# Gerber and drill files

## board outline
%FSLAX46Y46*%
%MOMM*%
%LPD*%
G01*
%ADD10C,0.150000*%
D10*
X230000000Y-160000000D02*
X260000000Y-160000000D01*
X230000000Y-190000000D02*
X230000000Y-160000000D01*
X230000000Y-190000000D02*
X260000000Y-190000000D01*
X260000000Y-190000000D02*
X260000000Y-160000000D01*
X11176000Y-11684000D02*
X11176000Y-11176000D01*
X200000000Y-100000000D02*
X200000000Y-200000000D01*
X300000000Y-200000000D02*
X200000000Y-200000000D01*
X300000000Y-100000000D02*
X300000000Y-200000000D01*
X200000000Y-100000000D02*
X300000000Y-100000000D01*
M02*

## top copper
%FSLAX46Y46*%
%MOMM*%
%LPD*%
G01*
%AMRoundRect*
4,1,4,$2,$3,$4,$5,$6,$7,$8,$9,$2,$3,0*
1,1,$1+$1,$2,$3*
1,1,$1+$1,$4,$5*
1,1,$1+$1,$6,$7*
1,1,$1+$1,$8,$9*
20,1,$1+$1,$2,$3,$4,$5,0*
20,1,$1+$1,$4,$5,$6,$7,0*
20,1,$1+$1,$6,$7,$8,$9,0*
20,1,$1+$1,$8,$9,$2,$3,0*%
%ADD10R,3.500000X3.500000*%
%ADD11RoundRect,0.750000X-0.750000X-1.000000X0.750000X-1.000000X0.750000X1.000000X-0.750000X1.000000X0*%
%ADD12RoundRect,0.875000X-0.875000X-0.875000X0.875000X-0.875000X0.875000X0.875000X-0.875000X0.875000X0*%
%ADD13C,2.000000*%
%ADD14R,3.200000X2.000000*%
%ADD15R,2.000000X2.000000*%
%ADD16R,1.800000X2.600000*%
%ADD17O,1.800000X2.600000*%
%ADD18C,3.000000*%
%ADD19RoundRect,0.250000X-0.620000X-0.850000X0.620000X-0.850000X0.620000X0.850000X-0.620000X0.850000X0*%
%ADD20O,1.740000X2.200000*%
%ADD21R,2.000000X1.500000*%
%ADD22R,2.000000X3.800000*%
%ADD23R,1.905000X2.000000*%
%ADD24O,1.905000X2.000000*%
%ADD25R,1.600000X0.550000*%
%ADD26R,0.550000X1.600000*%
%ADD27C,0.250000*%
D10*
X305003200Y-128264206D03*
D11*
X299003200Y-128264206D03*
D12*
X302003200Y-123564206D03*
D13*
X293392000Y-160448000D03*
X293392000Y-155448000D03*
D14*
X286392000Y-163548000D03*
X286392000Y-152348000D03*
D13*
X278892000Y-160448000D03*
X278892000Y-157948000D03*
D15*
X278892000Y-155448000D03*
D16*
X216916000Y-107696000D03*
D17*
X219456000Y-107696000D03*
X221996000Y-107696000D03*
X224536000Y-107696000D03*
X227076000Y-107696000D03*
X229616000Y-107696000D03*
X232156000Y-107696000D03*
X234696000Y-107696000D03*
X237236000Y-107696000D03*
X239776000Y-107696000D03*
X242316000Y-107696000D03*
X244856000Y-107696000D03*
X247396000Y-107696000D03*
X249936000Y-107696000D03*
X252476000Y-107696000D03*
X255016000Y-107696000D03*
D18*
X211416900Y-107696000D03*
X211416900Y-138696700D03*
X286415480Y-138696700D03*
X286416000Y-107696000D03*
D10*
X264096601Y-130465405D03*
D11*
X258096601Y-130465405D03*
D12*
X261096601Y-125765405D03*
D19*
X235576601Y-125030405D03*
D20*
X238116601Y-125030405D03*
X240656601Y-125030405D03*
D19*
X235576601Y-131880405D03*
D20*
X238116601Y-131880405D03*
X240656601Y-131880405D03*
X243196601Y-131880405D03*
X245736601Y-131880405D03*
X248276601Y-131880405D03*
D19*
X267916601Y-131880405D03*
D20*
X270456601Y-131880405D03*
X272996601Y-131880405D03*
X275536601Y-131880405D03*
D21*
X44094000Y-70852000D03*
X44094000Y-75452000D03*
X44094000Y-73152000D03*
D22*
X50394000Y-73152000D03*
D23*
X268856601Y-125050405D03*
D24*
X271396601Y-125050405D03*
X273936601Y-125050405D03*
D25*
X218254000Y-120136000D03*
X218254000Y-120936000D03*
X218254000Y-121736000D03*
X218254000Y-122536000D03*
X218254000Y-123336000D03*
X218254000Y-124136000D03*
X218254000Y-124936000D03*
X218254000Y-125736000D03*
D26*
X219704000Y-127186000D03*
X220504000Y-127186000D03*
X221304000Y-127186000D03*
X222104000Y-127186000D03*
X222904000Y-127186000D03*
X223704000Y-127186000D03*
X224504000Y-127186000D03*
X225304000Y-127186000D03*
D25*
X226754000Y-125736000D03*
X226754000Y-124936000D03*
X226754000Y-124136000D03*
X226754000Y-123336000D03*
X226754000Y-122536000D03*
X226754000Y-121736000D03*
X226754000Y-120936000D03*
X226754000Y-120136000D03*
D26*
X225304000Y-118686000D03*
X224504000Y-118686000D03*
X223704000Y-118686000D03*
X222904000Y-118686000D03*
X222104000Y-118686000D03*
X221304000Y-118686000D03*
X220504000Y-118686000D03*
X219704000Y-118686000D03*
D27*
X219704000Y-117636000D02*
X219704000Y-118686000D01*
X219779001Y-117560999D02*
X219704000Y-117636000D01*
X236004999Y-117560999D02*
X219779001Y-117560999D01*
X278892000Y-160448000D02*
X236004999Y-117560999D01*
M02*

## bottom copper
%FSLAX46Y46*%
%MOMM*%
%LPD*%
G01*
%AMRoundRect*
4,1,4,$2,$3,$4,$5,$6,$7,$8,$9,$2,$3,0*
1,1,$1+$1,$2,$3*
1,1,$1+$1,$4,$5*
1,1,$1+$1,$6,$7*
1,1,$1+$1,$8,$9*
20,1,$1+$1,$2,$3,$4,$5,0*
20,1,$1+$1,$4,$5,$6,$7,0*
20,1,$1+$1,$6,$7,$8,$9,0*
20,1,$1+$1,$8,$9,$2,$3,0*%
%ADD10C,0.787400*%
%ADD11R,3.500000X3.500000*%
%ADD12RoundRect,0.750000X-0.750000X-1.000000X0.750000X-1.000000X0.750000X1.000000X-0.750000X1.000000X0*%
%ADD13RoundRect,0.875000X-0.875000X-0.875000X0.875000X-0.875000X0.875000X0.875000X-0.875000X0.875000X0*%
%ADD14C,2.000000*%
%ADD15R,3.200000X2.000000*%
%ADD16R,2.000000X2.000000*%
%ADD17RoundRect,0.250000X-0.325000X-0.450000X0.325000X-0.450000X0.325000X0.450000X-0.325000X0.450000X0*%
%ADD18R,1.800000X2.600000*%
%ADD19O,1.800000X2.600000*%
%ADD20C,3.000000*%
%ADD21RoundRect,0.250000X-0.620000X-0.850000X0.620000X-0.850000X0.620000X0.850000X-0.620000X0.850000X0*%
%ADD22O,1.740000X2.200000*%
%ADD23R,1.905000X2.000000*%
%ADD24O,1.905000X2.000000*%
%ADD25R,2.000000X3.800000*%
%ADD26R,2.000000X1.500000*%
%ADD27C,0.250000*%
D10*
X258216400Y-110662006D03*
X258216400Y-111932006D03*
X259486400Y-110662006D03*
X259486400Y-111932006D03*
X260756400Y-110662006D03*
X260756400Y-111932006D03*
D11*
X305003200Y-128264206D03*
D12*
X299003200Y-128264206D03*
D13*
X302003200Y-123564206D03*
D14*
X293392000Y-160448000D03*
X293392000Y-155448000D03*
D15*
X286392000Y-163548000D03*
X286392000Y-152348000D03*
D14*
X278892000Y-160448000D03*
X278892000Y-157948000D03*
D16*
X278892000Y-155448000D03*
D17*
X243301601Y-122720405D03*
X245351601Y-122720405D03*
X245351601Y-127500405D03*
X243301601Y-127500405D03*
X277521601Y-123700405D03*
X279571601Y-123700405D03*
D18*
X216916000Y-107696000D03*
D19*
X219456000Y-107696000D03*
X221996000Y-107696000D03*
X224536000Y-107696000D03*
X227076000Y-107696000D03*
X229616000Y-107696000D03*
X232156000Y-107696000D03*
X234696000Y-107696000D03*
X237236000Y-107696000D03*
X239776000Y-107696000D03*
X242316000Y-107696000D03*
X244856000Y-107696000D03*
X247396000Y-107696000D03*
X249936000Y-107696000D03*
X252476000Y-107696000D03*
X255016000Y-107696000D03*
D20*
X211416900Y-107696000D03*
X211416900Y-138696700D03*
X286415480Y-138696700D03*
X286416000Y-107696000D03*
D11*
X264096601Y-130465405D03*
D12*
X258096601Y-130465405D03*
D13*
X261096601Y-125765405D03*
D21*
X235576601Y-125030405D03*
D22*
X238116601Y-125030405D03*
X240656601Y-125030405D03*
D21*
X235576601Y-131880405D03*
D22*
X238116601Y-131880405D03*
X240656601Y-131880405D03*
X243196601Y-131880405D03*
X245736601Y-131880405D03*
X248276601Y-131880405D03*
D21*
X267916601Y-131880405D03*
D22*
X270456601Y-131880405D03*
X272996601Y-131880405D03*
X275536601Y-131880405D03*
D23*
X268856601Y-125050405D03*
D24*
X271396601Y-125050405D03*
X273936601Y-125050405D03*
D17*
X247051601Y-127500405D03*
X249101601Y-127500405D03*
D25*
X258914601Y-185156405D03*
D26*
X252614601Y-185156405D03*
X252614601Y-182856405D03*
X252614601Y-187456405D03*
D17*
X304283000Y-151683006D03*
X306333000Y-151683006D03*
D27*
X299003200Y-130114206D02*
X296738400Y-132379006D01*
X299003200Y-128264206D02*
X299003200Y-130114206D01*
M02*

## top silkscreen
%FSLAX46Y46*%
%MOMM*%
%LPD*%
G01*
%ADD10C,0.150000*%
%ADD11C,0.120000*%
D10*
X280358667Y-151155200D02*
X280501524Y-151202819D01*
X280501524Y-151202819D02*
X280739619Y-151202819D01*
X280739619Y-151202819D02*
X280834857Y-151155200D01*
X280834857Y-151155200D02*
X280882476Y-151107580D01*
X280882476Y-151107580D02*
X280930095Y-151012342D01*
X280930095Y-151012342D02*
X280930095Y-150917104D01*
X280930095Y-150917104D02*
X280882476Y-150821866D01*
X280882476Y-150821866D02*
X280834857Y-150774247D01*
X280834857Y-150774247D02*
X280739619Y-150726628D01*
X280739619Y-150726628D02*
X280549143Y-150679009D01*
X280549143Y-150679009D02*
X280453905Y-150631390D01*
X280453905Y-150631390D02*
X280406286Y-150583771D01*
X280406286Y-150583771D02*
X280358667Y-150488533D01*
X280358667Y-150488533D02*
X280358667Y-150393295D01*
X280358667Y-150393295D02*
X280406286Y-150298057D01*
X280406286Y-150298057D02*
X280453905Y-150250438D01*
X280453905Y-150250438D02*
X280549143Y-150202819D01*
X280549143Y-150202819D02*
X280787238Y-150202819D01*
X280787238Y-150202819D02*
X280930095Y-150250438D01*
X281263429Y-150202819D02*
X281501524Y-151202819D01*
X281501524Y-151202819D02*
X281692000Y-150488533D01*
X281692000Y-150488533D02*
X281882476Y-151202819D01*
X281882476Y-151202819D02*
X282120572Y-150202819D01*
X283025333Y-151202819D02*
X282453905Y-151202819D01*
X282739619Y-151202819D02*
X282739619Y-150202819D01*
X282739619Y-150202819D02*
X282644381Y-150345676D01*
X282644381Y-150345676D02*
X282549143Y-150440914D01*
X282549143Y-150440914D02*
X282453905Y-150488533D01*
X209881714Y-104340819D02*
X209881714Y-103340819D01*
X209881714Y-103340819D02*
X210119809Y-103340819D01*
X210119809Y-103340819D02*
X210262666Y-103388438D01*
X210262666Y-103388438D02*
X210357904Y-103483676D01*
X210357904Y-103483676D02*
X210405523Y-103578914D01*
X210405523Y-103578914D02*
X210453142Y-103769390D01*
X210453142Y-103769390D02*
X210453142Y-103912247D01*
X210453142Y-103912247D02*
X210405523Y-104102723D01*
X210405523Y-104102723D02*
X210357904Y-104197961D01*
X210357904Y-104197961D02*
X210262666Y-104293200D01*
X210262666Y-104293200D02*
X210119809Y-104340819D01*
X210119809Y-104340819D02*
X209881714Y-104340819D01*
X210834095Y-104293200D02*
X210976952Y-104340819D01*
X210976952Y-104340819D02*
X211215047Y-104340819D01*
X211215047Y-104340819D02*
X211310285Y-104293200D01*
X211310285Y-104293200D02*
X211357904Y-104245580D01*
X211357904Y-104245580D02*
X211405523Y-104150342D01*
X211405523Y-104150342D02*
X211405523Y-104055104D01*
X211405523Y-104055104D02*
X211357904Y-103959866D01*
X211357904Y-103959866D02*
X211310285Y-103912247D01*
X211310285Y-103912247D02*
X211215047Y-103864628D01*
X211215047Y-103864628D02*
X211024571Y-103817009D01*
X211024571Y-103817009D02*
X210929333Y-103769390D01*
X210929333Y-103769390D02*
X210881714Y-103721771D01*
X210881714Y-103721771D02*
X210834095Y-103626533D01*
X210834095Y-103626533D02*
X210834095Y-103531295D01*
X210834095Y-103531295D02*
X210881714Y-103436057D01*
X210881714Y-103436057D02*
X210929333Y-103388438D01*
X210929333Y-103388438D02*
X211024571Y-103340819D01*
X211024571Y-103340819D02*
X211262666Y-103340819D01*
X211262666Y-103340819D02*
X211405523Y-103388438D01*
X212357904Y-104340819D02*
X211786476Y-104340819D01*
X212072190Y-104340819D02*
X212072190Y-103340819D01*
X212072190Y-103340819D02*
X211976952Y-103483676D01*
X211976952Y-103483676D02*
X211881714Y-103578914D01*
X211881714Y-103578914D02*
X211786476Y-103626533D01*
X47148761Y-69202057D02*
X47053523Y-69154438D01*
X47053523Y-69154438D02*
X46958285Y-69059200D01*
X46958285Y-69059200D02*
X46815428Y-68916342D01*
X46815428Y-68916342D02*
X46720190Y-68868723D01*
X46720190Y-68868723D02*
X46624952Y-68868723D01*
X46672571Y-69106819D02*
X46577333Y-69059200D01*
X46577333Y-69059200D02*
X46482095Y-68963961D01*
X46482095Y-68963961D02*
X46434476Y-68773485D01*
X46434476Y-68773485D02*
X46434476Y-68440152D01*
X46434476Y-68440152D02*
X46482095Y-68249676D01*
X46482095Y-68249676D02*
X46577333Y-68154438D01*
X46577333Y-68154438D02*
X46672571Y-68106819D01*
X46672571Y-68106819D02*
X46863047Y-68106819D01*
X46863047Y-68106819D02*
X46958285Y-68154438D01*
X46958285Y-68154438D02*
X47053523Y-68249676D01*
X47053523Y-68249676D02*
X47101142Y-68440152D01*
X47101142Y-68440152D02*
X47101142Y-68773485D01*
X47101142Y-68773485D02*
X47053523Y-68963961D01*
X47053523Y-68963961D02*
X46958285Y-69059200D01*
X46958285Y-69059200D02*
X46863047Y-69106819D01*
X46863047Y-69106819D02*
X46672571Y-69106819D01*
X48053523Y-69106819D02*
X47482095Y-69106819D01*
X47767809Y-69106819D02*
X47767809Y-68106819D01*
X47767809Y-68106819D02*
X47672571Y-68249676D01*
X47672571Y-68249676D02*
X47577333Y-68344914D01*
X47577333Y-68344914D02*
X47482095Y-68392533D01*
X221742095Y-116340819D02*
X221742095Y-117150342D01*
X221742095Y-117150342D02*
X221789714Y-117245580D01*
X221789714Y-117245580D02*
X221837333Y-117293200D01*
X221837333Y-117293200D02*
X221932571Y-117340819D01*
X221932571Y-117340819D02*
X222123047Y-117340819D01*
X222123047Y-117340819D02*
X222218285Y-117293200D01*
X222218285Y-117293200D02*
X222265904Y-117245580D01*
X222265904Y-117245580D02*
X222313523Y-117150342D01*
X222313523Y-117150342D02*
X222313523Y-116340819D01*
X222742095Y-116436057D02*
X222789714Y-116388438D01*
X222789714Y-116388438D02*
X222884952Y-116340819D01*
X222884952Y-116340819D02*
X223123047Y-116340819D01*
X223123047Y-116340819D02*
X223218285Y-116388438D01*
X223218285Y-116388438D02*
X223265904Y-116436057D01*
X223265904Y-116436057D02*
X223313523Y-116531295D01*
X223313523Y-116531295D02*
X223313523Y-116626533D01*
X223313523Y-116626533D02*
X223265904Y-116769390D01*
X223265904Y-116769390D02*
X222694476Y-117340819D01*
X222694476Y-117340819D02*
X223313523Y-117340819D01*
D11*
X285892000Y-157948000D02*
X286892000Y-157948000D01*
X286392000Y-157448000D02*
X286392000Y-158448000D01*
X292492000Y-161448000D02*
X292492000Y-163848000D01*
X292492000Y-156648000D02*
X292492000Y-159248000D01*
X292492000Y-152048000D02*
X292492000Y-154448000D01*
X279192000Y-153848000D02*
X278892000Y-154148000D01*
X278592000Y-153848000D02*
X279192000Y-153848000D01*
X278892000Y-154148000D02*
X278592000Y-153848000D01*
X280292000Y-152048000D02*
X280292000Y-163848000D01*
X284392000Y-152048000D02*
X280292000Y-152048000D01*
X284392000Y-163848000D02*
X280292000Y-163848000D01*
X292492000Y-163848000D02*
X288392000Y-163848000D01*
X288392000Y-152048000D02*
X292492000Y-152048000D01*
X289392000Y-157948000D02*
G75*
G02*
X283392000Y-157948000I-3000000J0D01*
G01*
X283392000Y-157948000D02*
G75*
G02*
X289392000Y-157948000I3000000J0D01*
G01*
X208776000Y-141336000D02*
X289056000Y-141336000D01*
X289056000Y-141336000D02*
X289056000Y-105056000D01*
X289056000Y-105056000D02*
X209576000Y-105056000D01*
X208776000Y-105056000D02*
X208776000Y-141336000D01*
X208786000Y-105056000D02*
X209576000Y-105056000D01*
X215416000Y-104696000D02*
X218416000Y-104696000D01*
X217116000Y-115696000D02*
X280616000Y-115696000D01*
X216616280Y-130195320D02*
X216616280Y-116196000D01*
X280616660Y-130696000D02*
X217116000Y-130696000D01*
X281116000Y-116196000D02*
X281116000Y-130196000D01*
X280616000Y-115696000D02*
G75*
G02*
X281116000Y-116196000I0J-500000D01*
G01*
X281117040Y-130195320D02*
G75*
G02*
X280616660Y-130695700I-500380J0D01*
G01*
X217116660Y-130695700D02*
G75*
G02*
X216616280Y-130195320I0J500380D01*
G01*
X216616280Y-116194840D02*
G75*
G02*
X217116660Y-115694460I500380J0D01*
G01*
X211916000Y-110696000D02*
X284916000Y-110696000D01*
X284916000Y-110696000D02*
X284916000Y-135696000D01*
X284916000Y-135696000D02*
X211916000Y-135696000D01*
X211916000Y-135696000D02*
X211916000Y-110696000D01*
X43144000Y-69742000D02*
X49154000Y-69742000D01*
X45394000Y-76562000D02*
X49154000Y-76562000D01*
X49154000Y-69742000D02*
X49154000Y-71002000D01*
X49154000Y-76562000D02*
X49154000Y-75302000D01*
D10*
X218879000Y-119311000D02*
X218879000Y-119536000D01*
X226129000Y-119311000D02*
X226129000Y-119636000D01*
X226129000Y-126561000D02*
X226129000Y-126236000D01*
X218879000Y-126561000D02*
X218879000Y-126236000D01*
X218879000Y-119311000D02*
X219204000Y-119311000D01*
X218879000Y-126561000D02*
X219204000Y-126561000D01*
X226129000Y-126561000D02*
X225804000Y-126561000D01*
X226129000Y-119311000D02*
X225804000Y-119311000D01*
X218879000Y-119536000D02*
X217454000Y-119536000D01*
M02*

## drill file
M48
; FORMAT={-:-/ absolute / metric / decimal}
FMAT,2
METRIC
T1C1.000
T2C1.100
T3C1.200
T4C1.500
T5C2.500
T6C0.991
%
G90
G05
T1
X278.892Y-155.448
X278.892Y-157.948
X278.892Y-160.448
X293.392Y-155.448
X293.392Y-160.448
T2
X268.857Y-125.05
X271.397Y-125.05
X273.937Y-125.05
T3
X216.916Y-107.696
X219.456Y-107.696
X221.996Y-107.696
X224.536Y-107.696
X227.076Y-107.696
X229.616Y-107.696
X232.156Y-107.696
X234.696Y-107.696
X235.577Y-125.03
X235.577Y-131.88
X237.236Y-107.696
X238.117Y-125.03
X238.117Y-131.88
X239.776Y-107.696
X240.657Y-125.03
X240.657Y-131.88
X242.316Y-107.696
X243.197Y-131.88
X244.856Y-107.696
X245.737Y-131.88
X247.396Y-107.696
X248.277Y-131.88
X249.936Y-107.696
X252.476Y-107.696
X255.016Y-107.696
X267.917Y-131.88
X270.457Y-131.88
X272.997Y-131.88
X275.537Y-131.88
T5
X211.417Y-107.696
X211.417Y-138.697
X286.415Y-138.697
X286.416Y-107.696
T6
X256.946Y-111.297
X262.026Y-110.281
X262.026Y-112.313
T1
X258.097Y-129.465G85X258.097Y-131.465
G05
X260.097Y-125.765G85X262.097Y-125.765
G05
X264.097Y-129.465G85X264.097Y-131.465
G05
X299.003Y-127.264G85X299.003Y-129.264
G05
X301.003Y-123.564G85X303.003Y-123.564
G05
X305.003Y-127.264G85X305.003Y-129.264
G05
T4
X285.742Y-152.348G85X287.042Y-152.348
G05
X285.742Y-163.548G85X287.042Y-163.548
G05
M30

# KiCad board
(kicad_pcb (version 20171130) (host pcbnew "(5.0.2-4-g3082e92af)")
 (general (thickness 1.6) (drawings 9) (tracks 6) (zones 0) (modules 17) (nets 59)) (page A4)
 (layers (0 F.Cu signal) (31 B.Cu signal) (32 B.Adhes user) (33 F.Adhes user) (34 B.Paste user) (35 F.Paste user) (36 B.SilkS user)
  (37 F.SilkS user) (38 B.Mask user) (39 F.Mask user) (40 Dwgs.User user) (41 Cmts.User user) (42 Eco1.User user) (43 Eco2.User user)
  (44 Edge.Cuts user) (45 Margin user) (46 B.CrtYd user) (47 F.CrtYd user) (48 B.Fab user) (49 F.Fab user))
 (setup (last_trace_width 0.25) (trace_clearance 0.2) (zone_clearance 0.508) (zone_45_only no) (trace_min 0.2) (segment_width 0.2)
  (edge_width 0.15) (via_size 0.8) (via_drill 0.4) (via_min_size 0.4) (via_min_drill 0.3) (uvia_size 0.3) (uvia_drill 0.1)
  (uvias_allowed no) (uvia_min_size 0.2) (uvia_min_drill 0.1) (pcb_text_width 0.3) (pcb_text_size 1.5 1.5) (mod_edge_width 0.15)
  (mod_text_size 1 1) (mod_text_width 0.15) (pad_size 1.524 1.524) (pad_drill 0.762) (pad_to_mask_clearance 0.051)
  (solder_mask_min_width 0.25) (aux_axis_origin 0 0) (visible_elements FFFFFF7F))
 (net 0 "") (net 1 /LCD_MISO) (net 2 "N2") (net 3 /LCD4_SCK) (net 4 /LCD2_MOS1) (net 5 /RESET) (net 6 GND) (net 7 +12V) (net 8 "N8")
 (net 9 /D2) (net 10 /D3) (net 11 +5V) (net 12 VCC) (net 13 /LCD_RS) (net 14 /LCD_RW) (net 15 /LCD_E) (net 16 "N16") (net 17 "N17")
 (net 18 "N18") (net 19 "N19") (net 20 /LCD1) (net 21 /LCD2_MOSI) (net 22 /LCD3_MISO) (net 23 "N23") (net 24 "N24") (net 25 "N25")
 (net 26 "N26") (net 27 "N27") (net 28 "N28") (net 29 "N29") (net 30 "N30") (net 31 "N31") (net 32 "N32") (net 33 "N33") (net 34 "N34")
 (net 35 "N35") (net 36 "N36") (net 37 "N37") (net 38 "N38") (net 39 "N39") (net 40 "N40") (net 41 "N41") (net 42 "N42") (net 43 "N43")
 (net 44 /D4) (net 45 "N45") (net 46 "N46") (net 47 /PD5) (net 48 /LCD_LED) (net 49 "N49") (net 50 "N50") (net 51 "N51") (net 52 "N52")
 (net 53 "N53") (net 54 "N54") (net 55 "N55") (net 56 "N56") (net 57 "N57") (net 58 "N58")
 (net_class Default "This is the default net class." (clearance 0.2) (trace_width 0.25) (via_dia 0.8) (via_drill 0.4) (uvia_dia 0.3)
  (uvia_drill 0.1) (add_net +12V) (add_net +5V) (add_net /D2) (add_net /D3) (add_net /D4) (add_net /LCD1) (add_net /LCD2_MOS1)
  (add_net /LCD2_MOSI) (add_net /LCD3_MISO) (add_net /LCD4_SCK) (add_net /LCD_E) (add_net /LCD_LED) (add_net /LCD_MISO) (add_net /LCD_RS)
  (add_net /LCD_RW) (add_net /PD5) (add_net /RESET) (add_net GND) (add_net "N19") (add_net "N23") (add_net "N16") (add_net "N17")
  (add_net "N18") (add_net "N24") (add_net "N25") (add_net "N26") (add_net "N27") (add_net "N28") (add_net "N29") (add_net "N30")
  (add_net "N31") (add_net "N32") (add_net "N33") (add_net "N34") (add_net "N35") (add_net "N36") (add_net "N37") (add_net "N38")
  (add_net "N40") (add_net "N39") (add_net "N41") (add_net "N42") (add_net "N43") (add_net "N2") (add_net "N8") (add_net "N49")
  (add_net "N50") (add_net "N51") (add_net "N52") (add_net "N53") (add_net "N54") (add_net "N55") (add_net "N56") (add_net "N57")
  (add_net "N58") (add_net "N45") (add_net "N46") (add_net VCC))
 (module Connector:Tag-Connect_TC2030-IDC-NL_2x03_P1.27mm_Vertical (layer B.Cu) (at 259.4864 111.297006)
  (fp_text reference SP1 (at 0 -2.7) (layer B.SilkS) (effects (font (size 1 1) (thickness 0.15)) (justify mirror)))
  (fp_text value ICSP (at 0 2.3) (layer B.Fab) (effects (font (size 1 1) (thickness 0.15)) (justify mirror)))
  (pad "" np_thru_hole circle (at 2.54 1.016) (size 0.9906 0.9906) (drill 0.9906) (layers *.Cu *.Mask))
  (pad "" np_thru_hole circle (at 2.54 -1.016) (size 0.9906 0.9906) (drill 0.9906) (layers *.Cu *.Mask))
  (pad "" np_thru_hole circle (at -2.54 0) (size 0.9906 0.9906) (drill 0.9906) (layers *.Cu *.Mask))
  (pad 1 connect circle (at -1.27 -0.635) (size 0.7874 0.7874) (layers B.Cu B.Mask) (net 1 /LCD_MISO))
  (pad 2 connect circle (at -1.27 0.635) (size 0.7874 0.7874) (layers B.Cu B.Mask) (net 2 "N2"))
  (pad 3 connect circle (at 0 -0.635) (size 0.7874 0.7874) (layers B.Cu B.Mask) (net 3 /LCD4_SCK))
  (pad 4 connect circle (at 0 0.635) (size 0.7874 0.7874) (layers B.Cu B.Mask) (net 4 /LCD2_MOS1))
  (pad 5 connect circle (at 1.27 -0.635) (size 0.7874 0.7874) (layers B.Cu B.Mask) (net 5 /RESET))
  (pad 6 connect circle (at 1.27 0.635) (size 0.7874 0.7874) (layers B.Cu B.Mask) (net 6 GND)))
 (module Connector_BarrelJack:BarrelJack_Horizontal (layer B.Cu) (at 305.0032 128.264206)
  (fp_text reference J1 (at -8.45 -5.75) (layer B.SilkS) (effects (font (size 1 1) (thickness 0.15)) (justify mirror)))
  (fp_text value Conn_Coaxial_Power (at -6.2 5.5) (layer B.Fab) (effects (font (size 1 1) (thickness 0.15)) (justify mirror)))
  (pad 1 thru_hole rect (at 0 0) (size 3.5 3.5) (drill oval 1 3) (layers *.Cu *.Mask) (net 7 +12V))
  (pad 2 thru_hole roundrect (at -6 0) (size 3 3.5) (drill oval 1 3) (layers *.Cu *.Mask) (roundrect_rratio 0.25) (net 6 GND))
  (pad 3 thru_hole roundrect (at -3 -4.7) (size 3.5 3.5) (drill oval 3 1) (layers *.Cu *.Mask) (roundrect_rratio 0.25)))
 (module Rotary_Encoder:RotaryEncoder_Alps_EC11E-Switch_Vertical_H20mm (layer F.Cu) (at 278.892 155.448)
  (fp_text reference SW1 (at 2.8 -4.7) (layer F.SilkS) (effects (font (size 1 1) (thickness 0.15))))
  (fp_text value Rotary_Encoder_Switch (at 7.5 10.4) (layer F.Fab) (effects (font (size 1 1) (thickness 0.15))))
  (fp_line (start 7 2.5) (end 8 2.5) (layer F.SilkS) (width 0.12))
  (fp_line (start 7.5 2) (end 7.5 3) (layer F.SilkS) (width 0.12))
  (fp_line (start 13.6 6) (end 13.6 8.4) (layer F.SilkS) (width 0.12))
  (fp_line (start 13.6 1.2) (end 13.6 3.8) (layer F.SilkS) (width 0.12))
  (fp_line (start 13.6 -3.4) (end 13.6 -1) (layer F.SilkS) (width 0.12))
  (fp_line (start 0.3 -1.6) (end 0 -1.3) (layer F.SilkS) (width 0.12))
  (fp_line (start -0.3 -1.6) (end 0.3 -1.6) (layer F.SilkS) (width 0.12))
  (fp_line (start 0 -1.3) (end -0.3 -1.6) (layer F.SilkS) (width 0.12))
  (fp_line (start 1.4 -3.4) (end 1.4 8.4) (layer F.SilkS) (width 0.12))
  (fp_line (start 5.5 -3.4) (end 1.4 -3.4) (layer F.SilkS) (width 0.12))
  (fp_line (start 5.5 8.4) (end 1.4 8.4) (layer F.SilkS) (width 0.12))
  (fp_line (start 13.6 8.4) (end 9.5 8.4) (layer F.SilkS) (width 0.12))
  (fp_line (start 9.5 -3.4) (end 13.6 -3.4) (layer F.SilkS) (width 0.12))
  (fp_circle (center 7.5 2.5) (end 10.5 2.5) (layer F.SilkS) (width 0.12))
  (pad S1 thru_hole circle (at 14.5 5) (size 2 2) (drill 1) (layers *.Cu *.Mask) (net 6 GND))
  (pad S2 thru_hole circle (at 14.5 0) (size 2 2) (drill 1) (layers *.Cu *.Mask) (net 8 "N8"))
  (pad MP thru_hole rect (at 7.5 8.1) (size 3.2 2) (drill oval 2.8 1.5) (layers *.Cu *.Mask))
  (pad MP thru_hole rect (at 7.5 -3.1) (size 3.2 2) (drill oval 2.8 1.5) (layers *.Cu *.Mask))
  (pad B thru_hole circle (at 0 5) (size 2 2) (drill 1) (layers *.Cu *.Mask) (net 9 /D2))
  (pad C thru_hole circle (at 0 2.5) (size 2 2) (drill 1) (layers *.Cu *.Mask) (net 6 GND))
  (pad A thru_hole rect (at 0 0) (size 2 2) (drill 1) (layers *.Cu *.Mask) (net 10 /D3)))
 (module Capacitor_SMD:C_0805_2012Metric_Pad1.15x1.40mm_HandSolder (layer B.Cu) (at 244.326601 122.720405)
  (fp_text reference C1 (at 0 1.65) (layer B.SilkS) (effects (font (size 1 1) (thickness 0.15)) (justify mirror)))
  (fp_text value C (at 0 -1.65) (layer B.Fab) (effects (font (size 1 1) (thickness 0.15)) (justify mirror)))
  (pad 1 smd roundrect (at -1.025 0) (size 1.15 1.4) (layers B.Cu B.Paste B.Mask) (roundrect_rratio 0.217391) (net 7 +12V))
  (pad 2 smd roundrect (at 1.025 0) (size 1.15 1.4) (layers B.Cu B.Paste B.Mask) (roundrect_rratio 0.217391) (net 6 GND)))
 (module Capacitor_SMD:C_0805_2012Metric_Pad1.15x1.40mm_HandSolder (layer B.Cu) (at 244.326601 127.500405)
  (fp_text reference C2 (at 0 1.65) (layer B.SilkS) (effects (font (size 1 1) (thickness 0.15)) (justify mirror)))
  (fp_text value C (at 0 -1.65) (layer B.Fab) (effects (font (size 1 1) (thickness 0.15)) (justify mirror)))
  (pad 2 smd roundrect (at 1.025 0) (size 1.15 1.4) (layers B.Cu B.Paste B.Mask) (roundrect_rratio 0.217391) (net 6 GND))
  (pad 1 smd roundrect (at -1.025 0) (size 1.15 1.4) (layers B.Cu B.Paste B.Mask) (roundrect_rratio 0.217391) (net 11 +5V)))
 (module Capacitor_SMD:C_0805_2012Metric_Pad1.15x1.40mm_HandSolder (layer B.Cu) (at 278.546601 123.700405)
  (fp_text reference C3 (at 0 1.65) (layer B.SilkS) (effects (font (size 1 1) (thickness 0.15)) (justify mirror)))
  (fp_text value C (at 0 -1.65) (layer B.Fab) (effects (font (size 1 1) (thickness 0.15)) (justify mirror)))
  (pad 1 smd roundrect (at -1.025 0) (size 1.15 1.4) (layers B.Cu B.Paste B.Mask) (roundrect_rratio 0.217391) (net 6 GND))
  (pad 2 smd roundrect (at 1.025 0) (size 1.15 1.4) (layers B.Cu B.Paste B.Mask) (roundrect_rratio 0.217391) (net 11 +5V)))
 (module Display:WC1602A (layer F.Cu) (at 216.916 107.696)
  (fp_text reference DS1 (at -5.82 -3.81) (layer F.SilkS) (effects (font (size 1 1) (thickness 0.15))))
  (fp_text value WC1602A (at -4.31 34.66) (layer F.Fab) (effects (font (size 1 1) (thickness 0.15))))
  (fp_line (start -8.14 33.64) (end 72.14 33.64) (layer F.SilkS) (width 0.12))
  (fp_line (start 72.14 33.64) (end 72.14 -2.64) (layer F.SilkS) (width 0.12))
  (fp_line (start 72.14 -2.64) (end -7.34 -2.64) (layer F.SilkS) (width 0.12))
  (fp_line (start -8.14 -2.64) (end -8.14 33.64) (layer F.SilkS) (width 0.12))
  (fp_line (start -8.13 -2.64) (end -7.34 -2.64) (layer F.SilkS) (width 0.12))
  (fp_line (start -1.5 -3) (end 1.5 -3) (layer F.SilkS) (width 0.12))
  (fp_line (start 0.2 8) (end 63.7 8) (layer F.SilkS) (width 0.12))
  (fp_line (start -0.29972 22.49932) (end -0.29972 8.5) (layer F.SilkS) (width 0.12))
  (fp_line (start 63.70066 23) (end 0.2 23) (layer F.SilkS) (width 0.12))
  (fp_line (start 64.2 8.5) (end 64.2 22.5) (layer F.SilkS) (width 0.12))
  (fp_arc (start 63.7 8.5) (end 63.7 8) (angle 90) (layer F.SilkS) (width 0.12))
  (fp_arc (start 63.70066 22.49932) (end 64.20104 22.49932) (angle 90) (layer F.SilkS) (width 0.12))
  (fp_arc (start 0.20066 22.49932) (end 0.20066 22.9997) (angle 90) (layer F.SilkS) (width 0.12))
  (fp_arc (start 0.20066 8.49884) (end -0.29972 8.49884) (angle 90) (layer F.SilkS) (width 0.12))
  (fp_line (start -5 3) (end 68 3) (layer F.SilkS) (width 0.12))
  (fp_line (start 68 3) (end 68 28) (layer F.SilkS) (width 0.12))
  (fp_line (start 68 28) (end -5 28) (layer F.SilkS) (width 0.12))
  (fp_line (start -5 28) (end -5 3) (layer F.SilkS) (width 0.12))
  (pad 1 thru_hole rect (at 0 0) (size 1.8 2.6) (drill 1.2) (layers *.Cu *.Mask) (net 6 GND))
  (pad 2 thru_hole oval (at 2.54 0) (size 1.8 2.6) (drill 1.2) (layers *.Cu *.Mask) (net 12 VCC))
  (pad 3 thru_hole oval (at 5.08 0) (size 1.8 2.6) (drill 1.2) (layers *.Cu *.Mask) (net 12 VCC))
  (pad 4 thru_hole oval (at 7.62 0) (size 1.8 2.6) (drill 1.2) (layers *.Cu *.Mask) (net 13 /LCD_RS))
  (pad 5 thru_hole oval (at 10.16 0) (size 1.8 2.6) (drill 1.2) (layers *.Cu *.Mask) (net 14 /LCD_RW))
  (pad 6 thru_hole oval (at 12.7 0) (size 1.8 2.6) (drill 1.2) (layers *.Cu *.Mask) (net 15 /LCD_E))
  (pad 7 thru_hole oval (at 15.24 0) (size 1.8 2.6) (drill 1.2) (layers *.Cu *.Mask) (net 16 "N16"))
  (pad 8 thru_hole oval (at 17.78 0) (size 1.8 2.6) (drill 1.2) (layers *.Cu *.Mask) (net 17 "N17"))
  (pad 9 thru_hole oval (at 20.32 0) (size 1.8 2.6) (drill 1.2) (layers *.Cu *.Mask) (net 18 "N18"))
  (pad 10 thru_hole oval (at 22.86 0) (size 1.8 2.6) (drill 1.2) (layers *.Cu *.Mask) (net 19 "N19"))
  (pad 11 thru_hole oval (at 25.4 0) (size 1.8 2.6) (drill 1.2) (layers *.Cu *.Mask) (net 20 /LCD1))
  (pad 12 thru_hole oval (at 27.94 0) (size 1.8 2.6) (drill 1.2) (layers *.Cu *.Mask) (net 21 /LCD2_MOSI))
  (pad 13 thru_hole oval (at 30.48 0) (size 1.8 2.6) (drill 1.2) (layers *.Cu *.Mask) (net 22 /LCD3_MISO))
  (pad 14 thru_hole oval (at 33.02 0) (size 1.8 2.6) (drill 1.2) (layers *.Cu *.Mask) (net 3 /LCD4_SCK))
  (pad 15 thru_hole oval (at 35.56 0) (size 1.8 2.6) (drill 1.2) (layers *.Cu *.Mask) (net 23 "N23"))
  (pad 16 thru_hole oval (at 38.1 0) (size 1.8 2.6) (drill 1.2) (layers *.Cu *.Mask) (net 6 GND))
  (pad "" thru_hole circle (at -5.4991 0) (size 3 3) (drill 2.5) (layers *.Cu *.Mask))
  (pad "" thru_hole circle (at -5.4991 31.0007) (size 3 3) (drill 2.5) (layers *.Cu *.Mask))
  (pad "" thru_hole circle (at 69.49948 31.0007) (size 3 3) (drill 2.5) (layers *.Cu *.Mask))
  (pad "" thru_hole circle (at 69.5 0) (size 3 3) (drill 2.5) (layers *.Cu *.Mask)))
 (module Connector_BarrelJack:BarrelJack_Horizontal (layer B.Cu) (at 264.096601 130.465405)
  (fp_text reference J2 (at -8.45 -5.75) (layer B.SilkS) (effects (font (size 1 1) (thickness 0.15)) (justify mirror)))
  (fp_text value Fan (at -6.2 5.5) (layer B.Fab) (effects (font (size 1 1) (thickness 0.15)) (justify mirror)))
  (pad 1 thru_hole rect (at 0 0) (size 3.5 3.5) (drill oval 1 3) (layers *.Cu *.Mask) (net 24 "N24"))
  (pad 2 thru_hole roundrect (at -6 0) (size 3 3.5) (drill oval 1 3) (layers *.Cu *.Mask) (roundrect_rratio 0.25) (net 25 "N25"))
  (pad 3 thru_hole roundrect (at -3 -4.7) (size 3.5 3.5) (drill oval 3 1) (layers *.Cu *.Mask) (roundrect_rratio 0.25)))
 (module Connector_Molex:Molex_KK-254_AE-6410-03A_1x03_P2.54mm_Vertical (layer B.Cu) (at 235.576601 125.030405)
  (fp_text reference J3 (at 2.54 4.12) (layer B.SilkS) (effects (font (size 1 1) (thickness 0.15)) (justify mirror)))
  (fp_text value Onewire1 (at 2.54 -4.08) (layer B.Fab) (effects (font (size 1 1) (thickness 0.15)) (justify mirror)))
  (pad 1 thru_hole roundrect (at 0 0) (size 1.74 2.2) (drill 1.2) (layers *.Cu *.Mask) (roundrect_rratio 0.143678) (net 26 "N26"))
  (pad 2 thru_hole oval (at 2.54 0) (size 1.74 2.2) (drill 1.2) (layers *.Cu *.Mask) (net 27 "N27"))
  (pad 3 thru_hole oval (at 5.08 0) (size 1.74 2.2) (drill 1.2) (layers *.Cu *.Mask) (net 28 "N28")))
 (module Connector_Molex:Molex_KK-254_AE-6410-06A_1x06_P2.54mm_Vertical (layer B.Cu) (at 235.576601 131.880405)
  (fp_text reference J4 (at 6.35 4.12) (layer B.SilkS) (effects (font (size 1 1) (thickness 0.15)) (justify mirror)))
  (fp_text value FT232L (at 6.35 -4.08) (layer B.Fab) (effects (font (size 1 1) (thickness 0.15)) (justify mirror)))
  (pad 1 thru_hole roundrect (at 0 0) (size 1.74 2.2) (drill 1.2) (layers *.Cu *.Mask) (roundrect_rratio 0.143678) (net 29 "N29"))
  (pad 2 thru_hole oval (at 2.54 0) (size 1.74 2.2) (drill 1.2) (layers *.Cu *.Mask) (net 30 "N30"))
  (pad 3 thru_hole oval (at 5.08 0) (size 1.74 2.2) (drill 1.2) (layers *.Cu *.Mask) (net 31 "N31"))
  (pad 4 thru_hole oval (at 7.62 0) (size 1.74 2.2) (drill 1.2) (layers *.Cu *.Mask) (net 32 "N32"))
  (pad 5 thru_hole oval (at 10.16 0) (size 1.74 2.2) (drill 1.2) (layers *.Cu *.Mask) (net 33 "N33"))
  (pad 6 thru_hole oval (at 12.7 0) (size 1.74 2.2) (drill 1.2) (layers *.Cu *.Mask) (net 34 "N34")))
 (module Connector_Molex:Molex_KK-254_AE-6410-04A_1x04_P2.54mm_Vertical (layer B.Cu) (at 267.916601 131.880405)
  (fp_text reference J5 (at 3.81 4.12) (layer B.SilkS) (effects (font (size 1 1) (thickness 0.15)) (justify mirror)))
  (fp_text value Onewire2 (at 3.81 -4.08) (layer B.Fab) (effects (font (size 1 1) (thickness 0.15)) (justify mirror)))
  (pad 1 thru_hole roundrect (at 0 0) (size 1.74 2.2) (drill 1.2) (layers *.Cu *.Mask) (roundrect_rratio 0.143678) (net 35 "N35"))
  (pad 2 thru_hole oval (at 2.54 0) (size 1.74 2.2) (drill 1.2) (layers *.Cu *.Mask) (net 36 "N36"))
  (pad 3 thru_hole oval (at 5.08 0) (size 1.74 2.2) (drill 1.2) (layers *.Cu *.Mask) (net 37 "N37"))
  (pad 4 thru_hole oval (at 7.62 0) (size 1.74 2.2) (drill 1.2) (layers *.Cu *.Mask)))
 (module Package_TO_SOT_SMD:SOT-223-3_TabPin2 (layer F.Cu) (at 47.244 73.152)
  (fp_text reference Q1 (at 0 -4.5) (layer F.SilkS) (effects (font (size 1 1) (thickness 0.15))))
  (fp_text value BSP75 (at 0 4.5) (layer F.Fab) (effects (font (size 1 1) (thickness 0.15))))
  (fp_line (start -4.1 -3.41) (end 1.91 -3.41) (layer F.SilkS) (width 0.12))
  (fp_line (start -1.85 3.41) (end 1.91 3.41) (layer F.SilkS) (width 0.12))
  (fp_line (start 1.91 -3.41) (end 1.91 -2.15) (layer F.SilkS) (width 0.12))
  (fp_line (start 1.91 3.41) (end 1.91 2.15) (layer F.SilkS) (width 0.12))
  (pad 1 smd rect (at -3.15 -2.3) (size 2 1.5) (layers F.Cu F.Paste F.Mask) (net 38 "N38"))
  (pad 3 smd rect (at -3.15 2.3) (size 2 1.5) (layers F.Cu F.Paste F.Mask) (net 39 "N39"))
  (pad 2 smd rect (at -3.15 0) (size 2 1.5) (layers F.Cu F.Paste F.Mask) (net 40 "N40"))
  (pad 2 smd rect (at 3.15 0) (size 2 3.8) (layers F.Cu F.Paste F.Mask) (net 40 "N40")))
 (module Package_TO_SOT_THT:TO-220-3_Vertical (layer B.Cu) (at 268.856601 125.050405)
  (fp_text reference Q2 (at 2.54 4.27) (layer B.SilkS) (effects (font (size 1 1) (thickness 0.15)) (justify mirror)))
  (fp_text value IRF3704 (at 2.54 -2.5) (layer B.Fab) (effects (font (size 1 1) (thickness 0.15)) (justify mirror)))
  (pad 1 thru_hole rect (at 0 0) (size 1.905 2) (drill 1.1) (layers *.Cu *.Mask) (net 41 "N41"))
  (pad 2 thru_hole oval (at 2.54 0) (size 1.905 2) (drill 1.1) (layers *.Cu *.Mask) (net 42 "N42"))
  (pad 3 thru_hole oval (at 5.08 0) (size 1.905 2) (drill 1.1) (layers *.Cu *.Mask) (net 6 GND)))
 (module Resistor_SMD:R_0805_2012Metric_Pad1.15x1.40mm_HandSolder (layer B.Cu) (at 248.076601 127.500405)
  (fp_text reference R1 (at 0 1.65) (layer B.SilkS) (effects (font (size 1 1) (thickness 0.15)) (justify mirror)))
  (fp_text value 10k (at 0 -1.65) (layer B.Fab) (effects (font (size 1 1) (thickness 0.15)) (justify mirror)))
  (pad 1 smd roundrect (at -1.025 0) (size 1.15 1.4) (layers B.Cu B.Paste B.Mask) (roundrect_rratio 0.217391) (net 11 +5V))
  (pad 2 smd roundrect (at 1.025 0) (size 1.15 1.4) (layers B.Cu B.Paste B.Mask) (roundrect_rratio 0.217391) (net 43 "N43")))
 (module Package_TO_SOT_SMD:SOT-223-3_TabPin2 (layer B.Cu) (at 255.764601 185.156405)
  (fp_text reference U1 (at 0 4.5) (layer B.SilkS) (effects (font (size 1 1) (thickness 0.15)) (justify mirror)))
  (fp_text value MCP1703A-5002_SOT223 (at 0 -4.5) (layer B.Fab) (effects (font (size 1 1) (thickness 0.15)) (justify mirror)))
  (pad 2 smd rect (at 3.15 0) (size 2 3.8) (layers B.Cu B.Paste B.Mask) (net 6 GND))
  (pad 2 smd rect (at -3.15 0) (size 2 1.5) (layers B.Cu B.Paste B.Mask) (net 6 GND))
  (pad 3 smd rect (at -3.15 -2.3) (size 2 1.5) (layers B.Cu B.Paste B.Mask) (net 11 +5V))
  (pad 1 smd rect (at -3.15 2.3) (size 2 1.5) (layers B.Cu B.Paste B.Mask) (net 7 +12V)))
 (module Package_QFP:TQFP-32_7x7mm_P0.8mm (layer F.Cu) (at 222.504 122.936)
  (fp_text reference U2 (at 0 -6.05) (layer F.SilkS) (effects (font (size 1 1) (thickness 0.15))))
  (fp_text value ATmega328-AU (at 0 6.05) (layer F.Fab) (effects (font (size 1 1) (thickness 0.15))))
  (fp_line (start -3.625 -3.625) (end -3.625 -3.4) (layer F.SilkS) (width 0.15))
  (fp_line (start 3.625 -3.625) (end 3.625 -3.3) (layer F.SilkS) (width 0.15))
  (fp_line (start 3.625 3.625) (end 3.625 3.3) (layer F.SilkS) (width 0.15))
  (fp_line (start -3.625 3.625) (end -3.625 3.3) (layer F.SilkS) (width 0.15))
  (fp_line (start -3.625 -3.625) (end -3.3 -3.625) (layer F.SilkS) (width 0.15))
  (fp_line (start -3.625 3.625) (end -3.3 3.625) (layer F.SilkS) (width 0.15))
  (fp_line (start 3.625 3.625) (end 3.3 3.625) (layer F.SilkS) (width 0.15))
  (fp_line (start 3.625 -3.625) (end 3.3 -3.625) (layer F.SilkS) (width 0.15))
  (fp_line (start -3.625 -3.4) (end -5.05 -3.4) (layer F.SilkS) (width 0.15))
  (pad 1 smd rect (at -4.25 -2.8) (size 1.6 0.55) (layers F.Cu F.Paste F.Mask) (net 10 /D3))
  (pad 2 smd rect (at -4.25 -2) (size 1.6 0.55) (layers F.Cu F.Paste F.Mask) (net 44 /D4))
  (pad 3 smd rect (at -4.25 -1.2) (size 1.6 0.55) (layers F.Cu F.Paste F.Mask) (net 6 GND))
  (pad 4 smd rect (at -4.25 -0.4) (size 1.6 0.55) (layers F.Cu F.Paste F.Mask) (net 11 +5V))
  (pad 5 smd rect (at -4.25 0.4) (size 1.6 0.55) (layers F.Cu F.Paste F.Mask) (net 6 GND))
  (pad 6 smd rect (at -4.25 1.2) (size 1.6 0.55) (layers F.Cu F.Paste F.Mask) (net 11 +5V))
  (pad 7 smd rect (at -4.25 2) (size 1.6 0.55) (layers F.Cu F.Paste F.Mask) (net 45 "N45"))
  (pad 8 smd rect (at -4.25 2.8) (size 1.6 0.55) (layers F.Cu F.Paste F.Mask) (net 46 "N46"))
  (pad 9 smd rect (at -2.8 4.25 90) (size 1.6 0.55) (layers F.Cu F.Paste F.Mask) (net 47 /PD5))
  (pad 10 smd rect (at -2 4.25 90) (size 1.6 0.55) (layers F.Cu F.Paste F.Mask) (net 13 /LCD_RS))
  (pad 11 smd rect (at -1.2 4.25 90) (size 1.6 0.55) (layers F.Cu F.Paste F.Mask) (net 14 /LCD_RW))
  (pad 12 smd rect (at -0.4 4.25 90) (size 1.6 0.55) (layers F.Cu F.Paste F.Mask) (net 15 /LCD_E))
  (pad 13 smd rect (at 0.4 4.25 90) (size 1.6 0.55) (layers F.Cu F.Paste F.Mask) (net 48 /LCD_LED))
  (pad 14 smd rect (at 1.2 4.25 90) (size 1.6 0.55) (layers F.Cu F.Paste F.Mask) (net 20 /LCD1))
  (pad 15 smd rect (at 2 4.25 90) (size 1.6 0.55) (layers F.Cu F.Paste F.Mask) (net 21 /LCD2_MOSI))
  (pad 16 smd rect (at 2.8 4.25 90) (size 1.6 0.55) (layers F.Cu F.Paste F.Mask) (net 22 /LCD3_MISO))
  (pad 17 smd rect (at 4.25 2.8) (size 1.6 0.55) (layers F.Cu F.Paste F.Mask) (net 3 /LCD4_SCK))
  (pad 18 smd rect (at 4.25 2) (size 1.6 0.55) (layers F.Cu F.Paste F.Mask) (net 11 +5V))
  (pad 19 smd rect (at 4.25 1.2) (size 1.6 0.55) (layers F.Cu F.Paste F.Mask) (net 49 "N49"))
  (pad 20 smd rect (at 4.25 0.4) (size 1.6 0.55) (layers F.Cu F.Paste F.Mask) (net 11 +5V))
  (pad 21 smd rect (at 4.25 -0.4) (size 1.6 0.55) (layers F.Cu F.Paste F.Mask) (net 6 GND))
  (pad 22 smd rect (at 4.25 -1.2) (size 1.6 0.55) (layers F.Cu F.Paste F.Mask) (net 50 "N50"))
  (pad 23 smd rect (at 4.25 -2) (size 1.6 0.55) (layers F.Cu F.Paste F.Mask) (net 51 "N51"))
  (pad 24 smd rect (at 4.25 -2.8) (size 1.6 0.55) (layers F.Cu F.Paste F.Mask) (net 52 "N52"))
  (pad 25 smd rect (at 2.8 -4.25 90) (size 1.6 0.55) (layers F.Cu F.Paste F.Mask) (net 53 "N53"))
  (pad 26 smd rect (at 2 -4.25 90) (size 1.6 0.55) (layers F.Cu F.Paste F.Mask) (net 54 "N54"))
  (pad 27 smd rect (at 1.2 -4.25 90) (size 1.6 0.55) (layers F.Cu F.Paste F.Mask) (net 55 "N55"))
  (pad 28 smd rect (at 0.4 -4.25 90) (size 1.6 0.55) (layers F.Cu F.Paste F.Mask) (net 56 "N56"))
  (pad 29 smd rect (at -0.4 -4.25 90) (size 1.6 0.55) (layers F.Cu F.Paste F.Mask) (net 43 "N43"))
  (pad 30 smd rect (at -1.2 -4.25 90) (size 1.6 0.55) (layers F.Cu F.Paste F.Mask) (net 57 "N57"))
  (pad 31 smd rect (at -2 -4.25 90) (size 1.6 0.55) (layers F.Cu F.Paste F.Mask) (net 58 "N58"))
  (pad 32 smd rect (at -2.8 -4.25 90) (size 1.6 0.55) (layers F.Cu F.Paste F.Mask) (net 9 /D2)))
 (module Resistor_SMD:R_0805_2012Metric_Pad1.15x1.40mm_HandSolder (layer B.Cu) (at 305.308 151.683006)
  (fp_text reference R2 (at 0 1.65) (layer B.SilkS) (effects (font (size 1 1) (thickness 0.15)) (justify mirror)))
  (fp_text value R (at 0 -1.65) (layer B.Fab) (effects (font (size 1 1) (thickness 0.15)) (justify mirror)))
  (pad 1 smd roundrect (at -1.025 0) (size 1.15 1.4) (layers B.Cu B.Paste B.Mask) (roundrect_rratio 0.217391) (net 48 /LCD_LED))
  (pad 2 smd roundrect (at 1.025 0) (size 1.15 1.4) (layers B.Cu B.Paste B.Mask) (roundrect_rratio 0.217391) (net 23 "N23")))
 (gr_line (start 230 160) (end 260 160) (layer Edge.Cuts) (width 0.15))
 (gr_line (start 230 190) (end 230 160) (layer Edge.Cuts) (width 0.15))
 (gr_line (start 230 190) (end 260 190) (layer Edge.Cuts) (width 0.15))
 (gr_line (start 260 190) (end 260 160) (layer Edge.Cuts) (width 0.15))
 (gr_line (start 11.176 11.684) (end 11.176 11.176) (layer Edge.Cuts) (width 0.15))
 (gr_line (start 200 100) (end 200 200) (layer Edge.Cuts) (width 0.15))
 (gr_line (start 300 200) (end 200 200) (layer Edge.Cuts) (width 0.15))
 (gr_line (start 300 100) (end 300 200) (layer Edge.Cuts) (width 0.15))
 (gr_line (start 200 100) (end 300 100) (layer Edge.Cuts) (width 0.15))
 (segment (start 299.0032 130.114206) (end 296.7384 132.379006) (width 0.25) (layer B.Cu) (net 6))
 (segment (start 299.0032 128.264206) (end 299.0032 130.114206) (width 0.25) (layer B.Cu) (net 6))
 (segment (start 219.704 117.636) (end 219.704 118.686) (width 0.25) (layer F.Cu) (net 9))
 (segment (start 219.779001 117.560999) (end 219.704 117.636) (width 0.25) (layer F.Cu) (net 9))
 (segment (start 236.004999 117.560999) (end 219.779001 117.560999) (width 0.25) (layer F.Cu) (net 9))
 (segment (start 278.892 160.448) (end 236.004999 117.560999) (width 0.25) (layer F.Cu) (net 9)))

